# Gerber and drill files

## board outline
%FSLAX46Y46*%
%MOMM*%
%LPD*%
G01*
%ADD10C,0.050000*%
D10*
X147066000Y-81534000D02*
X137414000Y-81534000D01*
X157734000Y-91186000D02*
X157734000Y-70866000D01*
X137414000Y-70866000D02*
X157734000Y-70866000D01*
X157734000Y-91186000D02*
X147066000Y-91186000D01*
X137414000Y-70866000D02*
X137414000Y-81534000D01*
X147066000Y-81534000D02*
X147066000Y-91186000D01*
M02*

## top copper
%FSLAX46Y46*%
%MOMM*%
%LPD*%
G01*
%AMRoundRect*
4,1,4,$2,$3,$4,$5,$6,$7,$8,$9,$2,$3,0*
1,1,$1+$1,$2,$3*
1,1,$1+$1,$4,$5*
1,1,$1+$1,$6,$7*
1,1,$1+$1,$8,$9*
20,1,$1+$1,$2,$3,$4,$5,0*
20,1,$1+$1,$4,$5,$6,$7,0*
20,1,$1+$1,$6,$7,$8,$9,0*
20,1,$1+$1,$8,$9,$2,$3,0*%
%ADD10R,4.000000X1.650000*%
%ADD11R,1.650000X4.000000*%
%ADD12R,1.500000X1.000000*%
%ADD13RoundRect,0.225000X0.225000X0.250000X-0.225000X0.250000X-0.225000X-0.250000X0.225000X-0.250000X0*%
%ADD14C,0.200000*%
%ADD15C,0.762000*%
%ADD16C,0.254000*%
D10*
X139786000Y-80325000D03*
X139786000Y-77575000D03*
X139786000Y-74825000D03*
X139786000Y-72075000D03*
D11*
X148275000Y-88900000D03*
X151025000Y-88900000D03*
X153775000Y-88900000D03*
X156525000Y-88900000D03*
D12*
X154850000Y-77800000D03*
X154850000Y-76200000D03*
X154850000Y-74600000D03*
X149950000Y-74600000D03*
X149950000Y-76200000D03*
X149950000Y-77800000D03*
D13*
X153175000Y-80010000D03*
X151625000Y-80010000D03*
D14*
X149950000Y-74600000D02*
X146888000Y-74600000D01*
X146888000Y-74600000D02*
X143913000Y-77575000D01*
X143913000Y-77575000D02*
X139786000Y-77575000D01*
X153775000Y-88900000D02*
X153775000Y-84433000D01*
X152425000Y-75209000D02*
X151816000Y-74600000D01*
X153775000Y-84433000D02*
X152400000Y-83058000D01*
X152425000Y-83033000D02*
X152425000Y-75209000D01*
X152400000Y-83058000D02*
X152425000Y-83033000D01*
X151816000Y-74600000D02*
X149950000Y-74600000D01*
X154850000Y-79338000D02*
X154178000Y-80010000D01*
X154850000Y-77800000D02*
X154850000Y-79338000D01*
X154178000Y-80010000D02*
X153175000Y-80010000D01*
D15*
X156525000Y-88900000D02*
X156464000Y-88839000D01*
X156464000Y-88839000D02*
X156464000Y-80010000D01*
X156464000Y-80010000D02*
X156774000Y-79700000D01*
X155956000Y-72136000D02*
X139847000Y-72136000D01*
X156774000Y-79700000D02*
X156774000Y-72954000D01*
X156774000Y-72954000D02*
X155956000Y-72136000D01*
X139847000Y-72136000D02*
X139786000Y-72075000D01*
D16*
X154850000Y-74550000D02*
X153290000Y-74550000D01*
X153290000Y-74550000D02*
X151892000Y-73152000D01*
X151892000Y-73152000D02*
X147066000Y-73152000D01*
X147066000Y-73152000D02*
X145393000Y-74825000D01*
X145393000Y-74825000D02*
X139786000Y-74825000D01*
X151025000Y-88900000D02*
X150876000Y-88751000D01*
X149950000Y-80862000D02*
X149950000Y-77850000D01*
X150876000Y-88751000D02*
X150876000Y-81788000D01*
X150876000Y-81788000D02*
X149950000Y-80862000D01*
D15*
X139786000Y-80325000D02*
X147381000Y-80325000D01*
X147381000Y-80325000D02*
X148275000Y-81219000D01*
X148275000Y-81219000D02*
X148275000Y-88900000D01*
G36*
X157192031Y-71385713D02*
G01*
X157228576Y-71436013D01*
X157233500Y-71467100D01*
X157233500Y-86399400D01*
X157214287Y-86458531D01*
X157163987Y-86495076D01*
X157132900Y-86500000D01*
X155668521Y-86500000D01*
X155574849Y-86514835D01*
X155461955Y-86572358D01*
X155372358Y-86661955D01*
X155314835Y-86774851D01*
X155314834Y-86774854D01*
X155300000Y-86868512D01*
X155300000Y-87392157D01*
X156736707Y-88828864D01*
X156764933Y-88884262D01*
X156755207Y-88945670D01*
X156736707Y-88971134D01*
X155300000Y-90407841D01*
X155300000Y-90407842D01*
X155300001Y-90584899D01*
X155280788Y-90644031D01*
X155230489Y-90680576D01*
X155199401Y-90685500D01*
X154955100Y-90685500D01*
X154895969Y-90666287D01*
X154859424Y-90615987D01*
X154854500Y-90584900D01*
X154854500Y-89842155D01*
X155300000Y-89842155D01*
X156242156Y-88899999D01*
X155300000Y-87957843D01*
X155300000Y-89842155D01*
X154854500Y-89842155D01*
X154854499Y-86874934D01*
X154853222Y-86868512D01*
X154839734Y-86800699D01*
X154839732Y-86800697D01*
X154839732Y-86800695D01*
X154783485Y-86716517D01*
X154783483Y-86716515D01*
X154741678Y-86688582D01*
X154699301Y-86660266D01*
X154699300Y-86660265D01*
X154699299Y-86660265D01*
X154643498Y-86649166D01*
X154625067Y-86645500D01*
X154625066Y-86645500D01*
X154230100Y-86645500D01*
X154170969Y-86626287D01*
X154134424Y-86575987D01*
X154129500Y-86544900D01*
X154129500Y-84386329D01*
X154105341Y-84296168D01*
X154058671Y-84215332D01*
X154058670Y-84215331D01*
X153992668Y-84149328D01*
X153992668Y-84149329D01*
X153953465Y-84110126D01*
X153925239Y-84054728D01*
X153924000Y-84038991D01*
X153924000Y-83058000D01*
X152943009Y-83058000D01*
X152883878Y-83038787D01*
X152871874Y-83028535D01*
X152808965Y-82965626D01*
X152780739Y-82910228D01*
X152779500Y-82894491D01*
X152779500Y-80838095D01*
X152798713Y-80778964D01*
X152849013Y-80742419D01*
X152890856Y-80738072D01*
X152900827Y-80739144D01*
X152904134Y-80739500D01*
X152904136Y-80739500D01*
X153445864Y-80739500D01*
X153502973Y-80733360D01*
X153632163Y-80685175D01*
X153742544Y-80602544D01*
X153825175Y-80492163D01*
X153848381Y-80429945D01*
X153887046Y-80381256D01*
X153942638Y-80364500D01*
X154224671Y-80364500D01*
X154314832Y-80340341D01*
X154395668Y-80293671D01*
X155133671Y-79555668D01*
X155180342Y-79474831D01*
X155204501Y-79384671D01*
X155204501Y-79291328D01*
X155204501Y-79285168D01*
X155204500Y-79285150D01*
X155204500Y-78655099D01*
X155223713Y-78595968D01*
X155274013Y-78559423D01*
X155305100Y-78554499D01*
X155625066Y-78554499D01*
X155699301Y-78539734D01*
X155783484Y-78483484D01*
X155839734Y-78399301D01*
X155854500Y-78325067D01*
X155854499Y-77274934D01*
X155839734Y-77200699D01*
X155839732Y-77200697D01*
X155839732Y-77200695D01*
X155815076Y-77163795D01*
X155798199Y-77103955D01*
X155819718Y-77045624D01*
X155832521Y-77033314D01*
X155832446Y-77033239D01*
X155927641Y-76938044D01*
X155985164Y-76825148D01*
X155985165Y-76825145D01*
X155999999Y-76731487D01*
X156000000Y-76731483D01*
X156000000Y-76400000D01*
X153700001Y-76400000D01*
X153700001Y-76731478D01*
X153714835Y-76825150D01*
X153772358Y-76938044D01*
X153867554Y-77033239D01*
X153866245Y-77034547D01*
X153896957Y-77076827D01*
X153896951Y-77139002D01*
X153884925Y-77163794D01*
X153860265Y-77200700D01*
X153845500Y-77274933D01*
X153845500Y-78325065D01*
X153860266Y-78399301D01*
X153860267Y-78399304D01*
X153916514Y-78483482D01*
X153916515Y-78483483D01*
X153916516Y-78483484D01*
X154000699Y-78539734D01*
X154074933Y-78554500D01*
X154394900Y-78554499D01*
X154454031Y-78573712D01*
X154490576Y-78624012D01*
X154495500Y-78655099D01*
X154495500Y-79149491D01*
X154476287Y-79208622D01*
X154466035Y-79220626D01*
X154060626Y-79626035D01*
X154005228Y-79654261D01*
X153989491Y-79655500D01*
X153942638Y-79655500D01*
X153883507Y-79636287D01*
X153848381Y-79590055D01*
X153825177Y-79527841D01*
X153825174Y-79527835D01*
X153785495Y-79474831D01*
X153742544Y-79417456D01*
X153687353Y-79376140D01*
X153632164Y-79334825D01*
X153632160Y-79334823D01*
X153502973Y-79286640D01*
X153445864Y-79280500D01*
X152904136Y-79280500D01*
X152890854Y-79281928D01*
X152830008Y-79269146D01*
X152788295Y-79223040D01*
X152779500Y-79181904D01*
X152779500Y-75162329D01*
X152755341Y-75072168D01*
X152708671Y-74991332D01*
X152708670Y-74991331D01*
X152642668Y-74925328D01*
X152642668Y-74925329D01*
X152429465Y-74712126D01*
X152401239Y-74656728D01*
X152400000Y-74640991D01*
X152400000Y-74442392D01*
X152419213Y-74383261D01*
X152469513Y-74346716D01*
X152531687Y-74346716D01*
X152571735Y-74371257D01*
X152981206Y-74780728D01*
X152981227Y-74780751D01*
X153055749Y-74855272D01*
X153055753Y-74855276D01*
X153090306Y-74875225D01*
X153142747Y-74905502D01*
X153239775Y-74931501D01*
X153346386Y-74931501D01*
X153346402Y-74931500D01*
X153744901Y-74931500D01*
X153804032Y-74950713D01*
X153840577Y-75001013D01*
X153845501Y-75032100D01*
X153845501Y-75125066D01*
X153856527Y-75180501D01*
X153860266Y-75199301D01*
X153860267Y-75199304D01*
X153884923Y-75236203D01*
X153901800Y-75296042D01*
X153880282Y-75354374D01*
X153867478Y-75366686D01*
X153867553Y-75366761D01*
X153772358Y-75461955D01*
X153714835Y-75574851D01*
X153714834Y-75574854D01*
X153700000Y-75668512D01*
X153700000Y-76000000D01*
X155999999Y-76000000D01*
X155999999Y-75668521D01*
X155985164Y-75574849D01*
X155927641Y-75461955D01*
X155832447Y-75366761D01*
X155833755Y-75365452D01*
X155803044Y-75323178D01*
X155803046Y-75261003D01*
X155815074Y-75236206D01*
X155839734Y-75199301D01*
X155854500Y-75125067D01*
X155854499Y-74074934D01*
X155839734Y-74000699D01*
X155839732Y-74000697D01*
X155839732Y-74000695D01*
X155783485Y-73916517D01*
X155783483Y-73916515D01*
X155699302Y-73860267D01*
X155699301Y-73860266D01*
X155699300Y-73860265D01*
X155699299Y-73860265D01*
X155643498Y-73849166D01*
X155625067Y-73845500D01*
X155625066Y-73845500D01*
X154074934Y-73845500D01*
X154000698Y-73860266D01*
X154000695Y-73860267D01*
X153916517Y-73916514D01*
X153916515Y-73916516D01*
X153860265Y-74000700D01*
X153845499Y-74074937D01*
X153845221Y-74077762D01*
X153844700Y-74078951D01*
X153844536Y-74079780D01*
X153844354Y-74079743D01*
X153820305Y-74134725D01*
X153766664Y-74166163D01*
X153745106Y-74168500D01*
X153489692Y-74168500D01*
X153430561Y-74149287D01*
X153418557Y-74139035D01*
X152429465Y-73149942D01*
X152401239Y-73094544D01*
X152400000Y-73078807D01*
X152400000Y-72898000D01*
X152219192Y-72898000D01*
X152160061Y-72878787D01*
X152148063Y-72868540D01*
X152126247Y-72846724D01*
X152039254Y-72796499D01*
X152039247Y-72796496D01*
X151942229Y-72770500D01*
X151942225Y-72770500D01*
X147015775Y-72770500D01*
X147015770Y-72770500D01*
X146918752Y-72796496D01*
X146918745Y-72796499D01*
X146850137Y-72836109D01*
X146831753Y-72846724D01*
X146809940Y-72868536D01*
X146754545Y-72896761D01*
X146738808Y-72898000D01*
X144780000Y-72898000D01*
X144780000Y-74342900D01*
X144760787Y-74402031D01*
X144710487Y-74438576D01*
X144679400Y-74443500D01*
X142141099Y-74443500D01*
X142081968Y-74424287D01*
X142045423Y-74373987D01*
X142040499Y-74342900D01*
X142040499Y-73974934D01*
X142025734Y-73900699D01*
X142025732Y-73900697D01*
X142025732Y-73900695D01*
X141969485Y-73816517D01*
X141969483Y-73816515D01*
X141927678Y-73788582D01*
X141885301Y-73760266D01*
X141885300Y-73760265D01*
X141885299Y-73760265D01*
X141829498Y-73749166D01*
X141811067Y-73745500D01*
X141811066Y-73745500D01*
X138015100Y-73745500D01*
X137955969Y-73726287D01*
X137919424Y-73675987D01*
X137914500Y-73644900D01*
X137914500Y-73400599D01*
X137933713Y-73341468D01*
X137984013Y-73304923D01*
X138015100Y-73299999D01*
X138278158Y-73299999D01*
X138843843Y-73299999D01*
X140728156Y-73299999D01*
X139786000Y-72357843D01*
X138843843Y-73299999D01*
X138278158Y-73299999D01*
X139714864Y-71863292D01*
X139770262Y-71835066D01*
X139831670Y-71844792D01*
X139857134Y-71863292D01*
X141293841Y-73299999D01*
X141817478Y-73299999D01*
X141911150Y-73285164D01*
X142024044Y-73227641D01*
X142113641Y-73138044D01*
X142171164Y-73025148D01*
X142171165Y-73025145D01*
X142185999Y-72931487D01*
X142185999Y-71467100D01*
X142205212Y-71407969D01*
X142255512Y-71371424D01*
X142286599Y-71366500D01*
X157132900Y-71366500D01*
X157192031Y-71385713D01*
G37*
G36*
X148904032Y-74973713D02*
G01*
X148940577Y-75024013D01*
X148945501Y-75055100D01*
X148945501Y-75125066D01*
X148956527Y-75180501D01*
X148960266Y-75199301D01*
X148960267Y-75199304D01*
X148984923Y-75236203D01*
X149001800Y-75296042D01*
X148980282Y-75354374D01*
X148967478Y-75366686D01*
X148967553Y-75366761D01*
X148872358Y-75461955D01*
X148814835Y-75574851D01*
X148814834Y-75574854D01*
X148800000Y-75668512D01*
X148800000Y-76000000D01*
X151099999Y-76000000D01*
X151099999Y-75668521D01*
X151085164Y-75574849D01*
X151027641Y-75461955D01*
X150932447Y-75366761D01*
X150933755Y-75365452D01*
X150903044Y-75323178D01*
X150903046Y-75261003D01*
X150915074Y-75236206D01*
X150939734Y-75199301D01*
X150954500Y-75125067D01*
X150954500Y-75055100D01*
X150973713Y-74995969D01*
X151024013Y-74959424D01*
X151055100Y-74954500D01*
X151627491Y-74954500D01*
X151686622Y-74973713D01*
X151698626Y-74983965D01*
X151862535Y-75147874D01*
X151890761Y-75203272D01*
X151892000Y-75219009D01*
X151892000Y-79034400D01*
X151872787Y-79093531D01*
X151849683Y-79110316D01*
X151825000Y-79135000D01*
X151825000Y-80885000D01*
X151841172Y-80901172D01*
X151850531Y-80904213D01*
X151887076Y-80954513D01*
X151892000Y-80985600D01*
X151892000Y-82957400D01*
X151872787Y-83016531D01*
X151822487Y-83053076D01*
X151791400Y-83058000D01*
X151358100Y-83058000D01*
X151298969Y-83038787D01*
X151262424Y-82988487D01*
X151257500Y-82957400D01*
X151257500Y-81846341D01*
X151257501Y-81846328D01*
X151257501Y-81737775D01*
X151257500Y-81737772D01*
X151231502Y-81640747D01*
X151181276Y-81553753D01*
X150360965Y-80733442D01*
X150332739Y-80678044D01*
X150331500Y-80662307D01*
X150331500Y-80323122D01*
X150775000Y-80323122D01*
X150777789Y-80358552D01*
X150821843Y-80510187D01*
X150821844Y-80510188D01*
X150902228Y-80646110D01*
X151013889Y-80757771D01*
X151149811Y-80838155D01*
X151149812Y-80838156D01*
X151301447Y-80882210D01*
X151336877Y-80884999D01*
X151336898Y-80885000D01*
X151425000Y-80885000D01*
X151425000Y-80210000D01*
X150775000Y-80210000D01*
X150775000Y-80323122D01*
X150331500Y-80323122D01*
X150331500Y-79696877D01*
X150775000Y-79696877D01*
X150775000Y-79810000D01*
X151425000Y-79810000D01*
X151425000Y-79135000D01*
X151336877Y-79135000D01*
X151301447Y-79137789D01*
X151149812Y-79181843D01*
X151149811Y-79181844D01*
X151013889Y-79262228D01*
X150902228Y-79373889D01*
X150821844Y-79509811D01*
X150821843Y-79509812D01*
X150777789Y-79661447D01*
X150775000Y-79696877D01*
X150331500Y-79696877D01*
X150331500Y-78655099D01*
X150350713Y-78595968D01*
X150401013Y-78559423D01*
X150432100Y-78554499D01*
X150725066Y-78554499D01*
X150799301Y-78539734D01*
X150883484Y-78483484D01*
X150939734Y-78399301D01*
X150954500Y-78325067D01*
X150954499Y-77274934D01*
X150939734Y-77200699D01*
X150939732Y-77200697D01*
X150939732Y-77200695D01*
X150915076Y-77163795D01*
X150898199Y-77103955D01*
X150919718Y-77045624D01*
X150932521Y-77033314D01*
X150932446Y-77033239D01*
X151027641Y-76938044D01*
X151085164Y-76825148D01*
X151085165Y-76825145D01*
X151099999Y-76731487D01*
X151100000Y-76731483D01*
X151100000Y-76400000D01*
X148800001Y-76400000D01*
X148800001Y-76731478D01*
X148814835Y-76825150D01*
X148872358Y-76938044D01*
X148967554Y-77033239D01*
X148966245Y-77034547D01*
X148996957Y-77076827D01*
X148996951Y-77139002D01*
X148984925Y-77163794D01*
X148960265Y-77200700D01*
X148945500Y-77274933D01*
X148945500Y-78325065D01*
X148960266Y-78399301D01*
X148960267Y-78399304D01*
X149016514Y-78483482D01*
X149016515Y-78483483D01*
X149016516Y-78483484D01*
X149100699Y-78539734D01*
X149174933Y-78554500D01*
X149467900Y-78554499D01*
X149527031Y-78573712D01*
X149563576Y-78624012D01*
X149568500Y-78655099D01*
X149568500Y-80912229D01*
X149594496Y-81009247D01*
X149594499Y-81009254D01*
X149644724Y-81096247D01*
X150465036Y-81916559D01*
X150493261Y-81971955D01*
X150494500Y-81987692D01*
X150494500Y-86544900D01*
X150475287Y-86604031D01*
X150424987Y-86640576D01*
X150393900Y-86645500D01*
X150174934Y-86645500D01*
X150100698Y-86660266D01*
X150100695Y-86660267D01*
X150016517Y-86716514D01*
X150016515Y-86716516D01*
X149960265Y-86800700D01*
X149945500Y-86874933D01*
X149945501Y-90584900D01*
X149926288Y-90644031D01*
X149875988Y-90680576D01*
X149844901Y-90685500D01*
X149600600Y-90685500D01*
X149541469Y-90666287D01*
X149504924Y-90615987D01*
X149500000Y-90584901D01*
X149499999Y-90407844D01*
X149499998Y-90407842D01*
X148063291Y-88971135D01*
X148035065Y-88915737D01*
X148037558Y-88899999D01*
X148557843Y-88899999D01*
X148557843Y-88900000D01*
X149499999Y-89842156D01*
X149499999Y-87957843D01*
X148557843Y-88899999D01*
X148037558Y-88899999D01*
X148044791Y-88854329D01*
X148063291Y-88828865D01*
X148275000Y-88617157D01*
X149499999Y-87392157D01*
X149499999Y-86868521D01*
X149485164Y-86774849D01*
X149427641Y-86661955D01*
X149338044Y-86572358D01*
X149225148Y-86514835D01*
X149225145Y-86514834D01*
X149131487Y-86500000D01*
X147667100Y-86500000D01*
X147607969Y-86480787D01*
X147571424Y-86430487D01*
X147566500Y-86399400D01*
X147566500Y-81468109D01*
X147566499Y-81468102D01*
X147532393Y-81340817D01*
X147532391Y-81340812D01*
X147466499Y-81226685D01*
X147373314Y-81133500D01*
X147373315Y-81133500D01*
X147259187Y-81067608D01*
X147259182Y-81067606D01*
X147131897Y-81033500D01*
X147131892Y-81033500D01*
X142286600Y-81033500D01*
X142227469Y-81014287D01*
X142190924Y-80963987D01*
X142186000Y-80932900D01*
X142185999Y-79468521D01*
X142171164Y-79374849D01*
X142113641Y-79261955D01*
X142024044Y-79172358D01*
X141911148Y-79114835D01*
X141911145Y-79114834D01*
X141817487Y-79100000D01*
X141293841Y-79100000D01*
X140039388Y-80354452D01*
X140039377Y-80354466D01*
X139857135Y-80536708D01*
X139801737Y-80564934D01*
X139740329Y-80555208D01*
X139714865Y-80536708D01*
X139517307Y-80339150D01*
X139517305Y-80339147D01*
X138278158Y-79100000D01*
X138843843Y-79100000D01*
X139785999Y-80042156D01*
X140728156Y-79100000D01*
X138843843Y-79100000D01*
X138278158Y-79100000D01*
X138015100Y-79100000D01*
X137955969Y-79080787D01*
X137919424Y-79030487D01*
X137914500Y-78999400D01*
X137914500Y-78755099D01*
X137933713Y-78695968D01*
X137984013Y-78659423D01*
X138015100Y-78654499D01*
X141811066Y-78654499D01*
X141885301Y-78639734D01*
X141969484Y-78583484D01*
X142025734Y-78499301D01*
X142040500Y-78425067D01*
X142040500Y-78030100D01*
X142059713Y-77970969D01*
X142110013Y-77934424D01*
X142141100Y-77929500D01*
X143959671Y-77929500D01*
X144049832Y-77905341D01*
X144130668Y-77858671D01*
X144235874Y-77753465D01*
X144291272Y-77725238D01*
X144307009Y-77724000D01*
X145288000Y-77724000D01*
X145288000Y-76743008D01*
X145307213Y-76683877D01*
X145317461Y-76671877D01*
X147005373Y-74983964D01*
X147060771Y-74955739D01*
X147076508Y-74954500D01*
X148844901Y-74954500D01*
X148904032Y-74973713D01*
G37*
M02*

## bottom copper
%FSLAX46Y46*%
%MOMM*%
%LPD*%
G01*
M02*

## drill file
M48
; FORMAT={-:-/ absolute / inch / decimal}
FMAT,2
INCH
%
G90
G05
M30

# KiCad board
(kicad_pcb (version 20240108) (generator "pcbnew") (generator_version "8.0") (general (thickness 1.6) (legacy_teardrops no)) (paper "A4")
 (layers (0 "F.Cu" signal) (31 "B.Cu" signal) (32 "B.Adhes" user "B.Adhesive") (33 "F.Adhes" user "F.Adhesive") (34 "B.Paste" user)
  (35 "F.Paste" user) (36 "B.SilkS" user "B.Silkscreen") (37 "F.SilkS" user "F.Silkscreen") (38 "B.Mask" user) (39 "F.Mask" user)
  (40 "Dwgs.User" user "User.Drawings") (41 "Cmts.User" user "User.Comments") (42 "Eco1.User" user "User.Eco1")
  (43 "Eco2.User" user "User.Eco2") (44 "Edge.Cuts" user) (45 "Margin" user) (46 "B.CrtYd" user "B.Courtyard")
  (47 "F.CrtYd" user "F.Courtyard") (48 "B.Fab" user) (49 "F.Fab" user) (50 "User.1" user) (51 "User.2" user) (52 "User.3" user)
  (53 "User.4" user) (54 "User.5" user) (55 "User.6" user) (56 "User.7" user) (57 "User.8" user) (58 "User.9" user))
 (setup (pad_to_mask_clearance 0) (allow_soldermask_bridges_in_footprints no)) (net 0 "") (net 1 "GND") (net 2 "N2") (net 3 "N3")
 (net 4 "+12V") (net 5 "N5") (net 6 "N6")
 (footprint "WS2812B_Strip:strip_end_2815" (layer "F.Cu") (at 143.786 76.2 180)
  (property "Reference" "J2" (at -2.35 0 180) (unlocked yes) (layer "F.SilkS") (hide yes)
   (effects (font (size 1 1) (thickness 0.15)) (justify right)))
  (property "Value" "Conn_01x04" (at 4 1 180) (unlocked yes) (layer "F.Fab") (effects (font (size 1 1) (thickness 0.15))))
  (pad "1" smd rect (at 4 -4.125 180) (size 4 1.65) (layers "F.Cu" "F.Paste" "F.Mask") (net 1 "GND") (thermal_bridge_angle 45))
  (pad "2" smd rect (at 4 -1.375 180) (size 4 1.65) (layers "F.Cu" "F.Paste" "F.Mask") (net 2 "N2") (thermal_bridge_angle 45))
  (pad "3" smd rect (at 4 1.375 180) (size 4 1.65) (layers "F.Cu" "F.Paste" "F.Mask") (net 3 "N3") (thermal_bridge_angle 45))
  (pad "4" smd rect (at 4 4.125 180) (size 4 1.65) (layers "F.Cu" "F.Paste" "F.Mask") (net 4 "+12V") (thermal_bridge_angle 45)))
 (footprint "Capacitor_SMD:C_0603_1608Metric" (layer "F.Cu") (at 152.4 80.01 180)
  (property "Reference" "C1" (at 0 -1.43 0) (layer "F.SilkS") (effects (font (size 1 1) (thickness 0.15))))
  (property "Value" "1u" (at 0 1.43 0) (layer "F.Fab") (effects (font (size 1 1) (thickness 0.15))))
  (pad "1" smd roundrect (at -0.775 0 180) (size 0.9 0.95) (layers "F.Cu" "F.Paste" "F.Mask") (roundrect_rratio 0.25) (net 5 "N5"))
  (pad "2" smd roundrect (at 0.775 0 180) (size 0.9 0.95) (layers "F.Cu" "F.Paste" "F.Mask") (roundrect_rratio 0.25) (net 1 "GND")))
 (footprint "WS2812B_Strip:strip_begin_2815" (layer "F.Cu") (at 152.4 88.9 90)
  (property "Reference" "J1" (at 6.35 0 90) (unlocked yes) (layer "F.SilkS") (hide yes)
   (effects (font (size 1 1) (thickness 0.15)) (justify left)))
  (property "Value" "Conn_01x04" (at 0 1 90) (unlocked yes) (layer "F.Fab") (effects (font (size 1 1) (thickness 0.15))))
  (pad "1" smd rect (at 0 -4.125 90) (size 4 1.65) (layers "F.Cu" "F.Paste" "F.Mask") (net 1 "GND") (thermal_bridge_angle 45))
  (pad "2" smd rect (at 0 -1.375 90) (size 4 1.65) (layers "F.Cu" "F.Paste" "F.Mask") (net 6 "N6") (thermal_bridge_angle 45))
  (pad "3" smd rect (at 0 1.375 90) (size 4 1.65) (layers "F.Cu" "F.Paste" "F.Mask") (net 2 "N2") (thermal_bridge_angle 45))
  (pad "4" smd rect (at 0 4.125 90) (size 4 1.65) (layers "F.Cu" "F.Paste" "F.Mask") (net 4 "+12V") (thermal_bridge_angle 45)))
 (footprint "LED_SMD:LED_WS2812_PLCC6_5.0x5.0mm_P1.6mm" (layer "F.Cu") (at 152.4 76.2 180)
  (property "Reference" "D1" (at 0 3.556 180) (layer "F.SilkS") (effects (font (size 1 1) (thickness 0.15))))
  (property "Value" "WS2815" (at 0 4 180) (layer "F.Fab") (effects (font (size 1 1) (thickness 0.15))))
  (pad "1" smd rect (at -2.45 -1.6 180) (size 1.5 1) (layers "F.Cu" "F.Paste" "F.Mask") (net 5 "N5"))
  (pad "2" smd rect (at -2.45 0 180) (size 1.5 1) (layers "F.Cu" "F.Paste" "F.Mask") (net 4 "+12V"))
  (pad "3" smd rect (at -2.45 1.6 180) (size 1.5 1) (layers "F.Cu" "F.Paste" "F.Mask") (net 3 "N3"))
  (pad "4" smd rect (at 2.45 1.6 180) (size 1.5 1) (layers "F.Cu" "F.Paste" "F.Mask") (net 2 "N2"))
  (pad "5" smd rect (at 2.45 0 180) (size 1.5 1) (layers "F.Cu" "F.Paste" "F.Mask") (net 1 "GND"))
  (pad "6" smd rect (at 2.45 -1.6 180) (size 1.5 1) (layers "F.Cu" "F.Paste" "F.Mask") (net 6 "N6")))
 (gr_line (start 147.066 81.534) (end 137.414 81.534) (stroke (width 0.05) (type default)) (layer "Edge.Cuts"))
 (gr_line (start 157.734 91.186) (end 157.734 70.866) (stroke (width 0.05) (type default)) (layer "Edge.Cuts"))
 (gr_line (start 137.414 70.866) (end 157.734 70.866) (stroke (width 0.05) (type default)) (layer "Edge.Cuts"))
 (gr_line (start 157.734 91.186) (end 147.066 91.186) (stroke (width 0.05) (type default)) (layer "Edge.Cuts"))
 (gr_line (start 137.414 70.866) (end 137.414 81.534) (stroke (width 0.05) (type default)) (layer "Edge.Cuts"))
 (gr_line (start 147.066 81.534) (end 147.066 91.186) (stroke (width 0.05) (type default)) (layer "Edge.Cuts"))
 (segment (start 143.913 77.575) (end 139.786 77.575) (width 0.2) (layer "F.Cu") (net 2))
 (segment (start 152.4 83.058) (end 152.425 83.033) (width 0.2) (layer "F.Cu") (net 2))
 (segment (start 153.775 88.9) (end 153.775 84.433) (width 0.2) (layer "F.Cu") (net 2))
 (segment (start 152.425 83.033) (end 152.425 75.209) (width 0.2) (layer "F.Cu") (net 2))
 (segment (start 146.888 74.6) (end 143.913 77.575) (width 0.2) (layer "F.Cu") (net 2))
 (segment (start 149.95 74.6) (end 146.888 74.6) (width 0.2) (layer "F.Cu") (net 2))
 (segment (start 151.816 74.6) (end 149.95 74.6) (width 0.2) (layer "F.Cu") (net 2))
 (segment (start 152.425 75.209) (end 151.816 74.6) (width 0.2) (layer "F.Cu") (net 2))
 (segment (start 153.775 84.433) (end 152.4 83.058) (width 0.2) (layer "F.Cu") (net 2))
 (segment (start 147.066 73.152) (end 145.393 74.825) (width 0.254) (layer "F.Cu") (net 3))
 (segment (start 145.393 74.825) (end 139.786 74.825) (width 0.254) (layer "F.Cu") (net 3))
 (segment (start 154.85 74.55) (end 153.29 74.55) (width 0.254) (layer "F.Cu") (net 3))
 (segment (start 153.29 74.55) (end 151.892 73.152) (width 0.254) (layer "F.Cu") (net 3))
 (segment (start 151.892 73.152) (end 147.066 73.152) (width 0.254) (layer "F.Cu") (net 3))
 (segment (start 147.381 80.325) (end 148.275 81.219) (width 0.762) (layer "F.Cu") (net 1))
 (segment (start 148.275 81.219) (end 148.275 88.9) (width 0.762) (layer "F.Cu") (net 1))
 (segment (start 139.786 80.325) (end 147.381 80.325) (width 0.762) (layer "F.Cu") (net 1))
 (segment (start 154.85 77.8) (end 154.85 79.338) (width 0.2) (layer "F.Cu") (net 5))
 (segment (start 154.178 80.01) (end 153.175 80.01) (width 0.2) (layer "F.Cu") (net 5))
 (segment (start 154.85 79.338) (end 154.178 80.01) (width 0.2) (layer "F.Cu") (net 5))
 (segment (start 150.876 88.751) (end 150.876 81.788) (width 0.254) (layer "F.Cu") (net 6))
 (segment (start 149.95 80.862) (end 149.95 77.85) (width 0.254) (layer "F.Cu") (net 6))
 (segment (start 150.876 81.788) (end 149.95 80.862) (width 0.254) (layer "F.Cu") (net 6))
 (segment (start 151.025 88.9) (end 150.876 88.751) (width 0.254) (layer "F.Cu") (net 6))
 (segment (start 156.464 80.01) (end 156.774 79.7) (width 0.762) (layer "F.Cu") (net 4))
 (segment (start 156.525 88.9) (end 156.464 88.839) (width 0.762) (layer "F.Cu") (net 4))
 (segment (start 156.464 88.839) (end 156.464 80.01) (width 0.762) (layer "F.Cu") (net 4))
 (segment (start 156.774 72.954) (end 155.956 72.136) (width 0.762) (layer "F.Cu") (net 4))
 (segment (start 139.847 72.136) (end 139.786 72.075) (width 0.762) (layer "F.Cu") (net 4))
 (segment (start 155.956 72.136) (end 139.847 72.136) (width 0.762) (layer "F.Cu") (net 4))
 (segment (start 156.774 79.7) (end 156.774 72.954) (width 0.762) (layer "F.Cu") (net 4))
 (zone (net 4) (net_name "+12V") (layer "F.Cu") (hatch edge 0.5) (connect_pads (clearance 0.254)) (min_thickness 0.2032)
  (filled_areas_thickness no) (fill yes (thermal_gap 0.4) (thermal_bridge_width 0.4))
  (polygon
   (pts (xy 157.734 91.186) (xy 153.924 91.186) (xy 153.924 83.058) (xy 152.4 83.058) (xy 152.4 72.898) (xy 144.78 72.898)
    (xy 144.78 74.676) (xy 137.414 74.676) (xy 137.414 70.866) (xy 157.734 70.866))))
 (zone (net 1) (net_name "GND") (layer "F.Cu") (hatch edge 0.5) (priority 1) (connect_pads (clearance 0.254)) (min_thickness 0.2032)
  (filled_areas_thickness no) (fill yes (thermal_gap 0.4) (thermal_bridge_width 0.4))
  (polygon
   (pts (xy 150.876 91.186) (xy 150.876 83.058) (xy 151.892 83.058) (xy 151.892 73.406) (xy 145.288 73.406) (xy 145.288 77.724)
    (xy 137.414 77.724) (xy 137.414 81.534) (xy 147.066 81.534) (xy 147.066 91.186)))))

